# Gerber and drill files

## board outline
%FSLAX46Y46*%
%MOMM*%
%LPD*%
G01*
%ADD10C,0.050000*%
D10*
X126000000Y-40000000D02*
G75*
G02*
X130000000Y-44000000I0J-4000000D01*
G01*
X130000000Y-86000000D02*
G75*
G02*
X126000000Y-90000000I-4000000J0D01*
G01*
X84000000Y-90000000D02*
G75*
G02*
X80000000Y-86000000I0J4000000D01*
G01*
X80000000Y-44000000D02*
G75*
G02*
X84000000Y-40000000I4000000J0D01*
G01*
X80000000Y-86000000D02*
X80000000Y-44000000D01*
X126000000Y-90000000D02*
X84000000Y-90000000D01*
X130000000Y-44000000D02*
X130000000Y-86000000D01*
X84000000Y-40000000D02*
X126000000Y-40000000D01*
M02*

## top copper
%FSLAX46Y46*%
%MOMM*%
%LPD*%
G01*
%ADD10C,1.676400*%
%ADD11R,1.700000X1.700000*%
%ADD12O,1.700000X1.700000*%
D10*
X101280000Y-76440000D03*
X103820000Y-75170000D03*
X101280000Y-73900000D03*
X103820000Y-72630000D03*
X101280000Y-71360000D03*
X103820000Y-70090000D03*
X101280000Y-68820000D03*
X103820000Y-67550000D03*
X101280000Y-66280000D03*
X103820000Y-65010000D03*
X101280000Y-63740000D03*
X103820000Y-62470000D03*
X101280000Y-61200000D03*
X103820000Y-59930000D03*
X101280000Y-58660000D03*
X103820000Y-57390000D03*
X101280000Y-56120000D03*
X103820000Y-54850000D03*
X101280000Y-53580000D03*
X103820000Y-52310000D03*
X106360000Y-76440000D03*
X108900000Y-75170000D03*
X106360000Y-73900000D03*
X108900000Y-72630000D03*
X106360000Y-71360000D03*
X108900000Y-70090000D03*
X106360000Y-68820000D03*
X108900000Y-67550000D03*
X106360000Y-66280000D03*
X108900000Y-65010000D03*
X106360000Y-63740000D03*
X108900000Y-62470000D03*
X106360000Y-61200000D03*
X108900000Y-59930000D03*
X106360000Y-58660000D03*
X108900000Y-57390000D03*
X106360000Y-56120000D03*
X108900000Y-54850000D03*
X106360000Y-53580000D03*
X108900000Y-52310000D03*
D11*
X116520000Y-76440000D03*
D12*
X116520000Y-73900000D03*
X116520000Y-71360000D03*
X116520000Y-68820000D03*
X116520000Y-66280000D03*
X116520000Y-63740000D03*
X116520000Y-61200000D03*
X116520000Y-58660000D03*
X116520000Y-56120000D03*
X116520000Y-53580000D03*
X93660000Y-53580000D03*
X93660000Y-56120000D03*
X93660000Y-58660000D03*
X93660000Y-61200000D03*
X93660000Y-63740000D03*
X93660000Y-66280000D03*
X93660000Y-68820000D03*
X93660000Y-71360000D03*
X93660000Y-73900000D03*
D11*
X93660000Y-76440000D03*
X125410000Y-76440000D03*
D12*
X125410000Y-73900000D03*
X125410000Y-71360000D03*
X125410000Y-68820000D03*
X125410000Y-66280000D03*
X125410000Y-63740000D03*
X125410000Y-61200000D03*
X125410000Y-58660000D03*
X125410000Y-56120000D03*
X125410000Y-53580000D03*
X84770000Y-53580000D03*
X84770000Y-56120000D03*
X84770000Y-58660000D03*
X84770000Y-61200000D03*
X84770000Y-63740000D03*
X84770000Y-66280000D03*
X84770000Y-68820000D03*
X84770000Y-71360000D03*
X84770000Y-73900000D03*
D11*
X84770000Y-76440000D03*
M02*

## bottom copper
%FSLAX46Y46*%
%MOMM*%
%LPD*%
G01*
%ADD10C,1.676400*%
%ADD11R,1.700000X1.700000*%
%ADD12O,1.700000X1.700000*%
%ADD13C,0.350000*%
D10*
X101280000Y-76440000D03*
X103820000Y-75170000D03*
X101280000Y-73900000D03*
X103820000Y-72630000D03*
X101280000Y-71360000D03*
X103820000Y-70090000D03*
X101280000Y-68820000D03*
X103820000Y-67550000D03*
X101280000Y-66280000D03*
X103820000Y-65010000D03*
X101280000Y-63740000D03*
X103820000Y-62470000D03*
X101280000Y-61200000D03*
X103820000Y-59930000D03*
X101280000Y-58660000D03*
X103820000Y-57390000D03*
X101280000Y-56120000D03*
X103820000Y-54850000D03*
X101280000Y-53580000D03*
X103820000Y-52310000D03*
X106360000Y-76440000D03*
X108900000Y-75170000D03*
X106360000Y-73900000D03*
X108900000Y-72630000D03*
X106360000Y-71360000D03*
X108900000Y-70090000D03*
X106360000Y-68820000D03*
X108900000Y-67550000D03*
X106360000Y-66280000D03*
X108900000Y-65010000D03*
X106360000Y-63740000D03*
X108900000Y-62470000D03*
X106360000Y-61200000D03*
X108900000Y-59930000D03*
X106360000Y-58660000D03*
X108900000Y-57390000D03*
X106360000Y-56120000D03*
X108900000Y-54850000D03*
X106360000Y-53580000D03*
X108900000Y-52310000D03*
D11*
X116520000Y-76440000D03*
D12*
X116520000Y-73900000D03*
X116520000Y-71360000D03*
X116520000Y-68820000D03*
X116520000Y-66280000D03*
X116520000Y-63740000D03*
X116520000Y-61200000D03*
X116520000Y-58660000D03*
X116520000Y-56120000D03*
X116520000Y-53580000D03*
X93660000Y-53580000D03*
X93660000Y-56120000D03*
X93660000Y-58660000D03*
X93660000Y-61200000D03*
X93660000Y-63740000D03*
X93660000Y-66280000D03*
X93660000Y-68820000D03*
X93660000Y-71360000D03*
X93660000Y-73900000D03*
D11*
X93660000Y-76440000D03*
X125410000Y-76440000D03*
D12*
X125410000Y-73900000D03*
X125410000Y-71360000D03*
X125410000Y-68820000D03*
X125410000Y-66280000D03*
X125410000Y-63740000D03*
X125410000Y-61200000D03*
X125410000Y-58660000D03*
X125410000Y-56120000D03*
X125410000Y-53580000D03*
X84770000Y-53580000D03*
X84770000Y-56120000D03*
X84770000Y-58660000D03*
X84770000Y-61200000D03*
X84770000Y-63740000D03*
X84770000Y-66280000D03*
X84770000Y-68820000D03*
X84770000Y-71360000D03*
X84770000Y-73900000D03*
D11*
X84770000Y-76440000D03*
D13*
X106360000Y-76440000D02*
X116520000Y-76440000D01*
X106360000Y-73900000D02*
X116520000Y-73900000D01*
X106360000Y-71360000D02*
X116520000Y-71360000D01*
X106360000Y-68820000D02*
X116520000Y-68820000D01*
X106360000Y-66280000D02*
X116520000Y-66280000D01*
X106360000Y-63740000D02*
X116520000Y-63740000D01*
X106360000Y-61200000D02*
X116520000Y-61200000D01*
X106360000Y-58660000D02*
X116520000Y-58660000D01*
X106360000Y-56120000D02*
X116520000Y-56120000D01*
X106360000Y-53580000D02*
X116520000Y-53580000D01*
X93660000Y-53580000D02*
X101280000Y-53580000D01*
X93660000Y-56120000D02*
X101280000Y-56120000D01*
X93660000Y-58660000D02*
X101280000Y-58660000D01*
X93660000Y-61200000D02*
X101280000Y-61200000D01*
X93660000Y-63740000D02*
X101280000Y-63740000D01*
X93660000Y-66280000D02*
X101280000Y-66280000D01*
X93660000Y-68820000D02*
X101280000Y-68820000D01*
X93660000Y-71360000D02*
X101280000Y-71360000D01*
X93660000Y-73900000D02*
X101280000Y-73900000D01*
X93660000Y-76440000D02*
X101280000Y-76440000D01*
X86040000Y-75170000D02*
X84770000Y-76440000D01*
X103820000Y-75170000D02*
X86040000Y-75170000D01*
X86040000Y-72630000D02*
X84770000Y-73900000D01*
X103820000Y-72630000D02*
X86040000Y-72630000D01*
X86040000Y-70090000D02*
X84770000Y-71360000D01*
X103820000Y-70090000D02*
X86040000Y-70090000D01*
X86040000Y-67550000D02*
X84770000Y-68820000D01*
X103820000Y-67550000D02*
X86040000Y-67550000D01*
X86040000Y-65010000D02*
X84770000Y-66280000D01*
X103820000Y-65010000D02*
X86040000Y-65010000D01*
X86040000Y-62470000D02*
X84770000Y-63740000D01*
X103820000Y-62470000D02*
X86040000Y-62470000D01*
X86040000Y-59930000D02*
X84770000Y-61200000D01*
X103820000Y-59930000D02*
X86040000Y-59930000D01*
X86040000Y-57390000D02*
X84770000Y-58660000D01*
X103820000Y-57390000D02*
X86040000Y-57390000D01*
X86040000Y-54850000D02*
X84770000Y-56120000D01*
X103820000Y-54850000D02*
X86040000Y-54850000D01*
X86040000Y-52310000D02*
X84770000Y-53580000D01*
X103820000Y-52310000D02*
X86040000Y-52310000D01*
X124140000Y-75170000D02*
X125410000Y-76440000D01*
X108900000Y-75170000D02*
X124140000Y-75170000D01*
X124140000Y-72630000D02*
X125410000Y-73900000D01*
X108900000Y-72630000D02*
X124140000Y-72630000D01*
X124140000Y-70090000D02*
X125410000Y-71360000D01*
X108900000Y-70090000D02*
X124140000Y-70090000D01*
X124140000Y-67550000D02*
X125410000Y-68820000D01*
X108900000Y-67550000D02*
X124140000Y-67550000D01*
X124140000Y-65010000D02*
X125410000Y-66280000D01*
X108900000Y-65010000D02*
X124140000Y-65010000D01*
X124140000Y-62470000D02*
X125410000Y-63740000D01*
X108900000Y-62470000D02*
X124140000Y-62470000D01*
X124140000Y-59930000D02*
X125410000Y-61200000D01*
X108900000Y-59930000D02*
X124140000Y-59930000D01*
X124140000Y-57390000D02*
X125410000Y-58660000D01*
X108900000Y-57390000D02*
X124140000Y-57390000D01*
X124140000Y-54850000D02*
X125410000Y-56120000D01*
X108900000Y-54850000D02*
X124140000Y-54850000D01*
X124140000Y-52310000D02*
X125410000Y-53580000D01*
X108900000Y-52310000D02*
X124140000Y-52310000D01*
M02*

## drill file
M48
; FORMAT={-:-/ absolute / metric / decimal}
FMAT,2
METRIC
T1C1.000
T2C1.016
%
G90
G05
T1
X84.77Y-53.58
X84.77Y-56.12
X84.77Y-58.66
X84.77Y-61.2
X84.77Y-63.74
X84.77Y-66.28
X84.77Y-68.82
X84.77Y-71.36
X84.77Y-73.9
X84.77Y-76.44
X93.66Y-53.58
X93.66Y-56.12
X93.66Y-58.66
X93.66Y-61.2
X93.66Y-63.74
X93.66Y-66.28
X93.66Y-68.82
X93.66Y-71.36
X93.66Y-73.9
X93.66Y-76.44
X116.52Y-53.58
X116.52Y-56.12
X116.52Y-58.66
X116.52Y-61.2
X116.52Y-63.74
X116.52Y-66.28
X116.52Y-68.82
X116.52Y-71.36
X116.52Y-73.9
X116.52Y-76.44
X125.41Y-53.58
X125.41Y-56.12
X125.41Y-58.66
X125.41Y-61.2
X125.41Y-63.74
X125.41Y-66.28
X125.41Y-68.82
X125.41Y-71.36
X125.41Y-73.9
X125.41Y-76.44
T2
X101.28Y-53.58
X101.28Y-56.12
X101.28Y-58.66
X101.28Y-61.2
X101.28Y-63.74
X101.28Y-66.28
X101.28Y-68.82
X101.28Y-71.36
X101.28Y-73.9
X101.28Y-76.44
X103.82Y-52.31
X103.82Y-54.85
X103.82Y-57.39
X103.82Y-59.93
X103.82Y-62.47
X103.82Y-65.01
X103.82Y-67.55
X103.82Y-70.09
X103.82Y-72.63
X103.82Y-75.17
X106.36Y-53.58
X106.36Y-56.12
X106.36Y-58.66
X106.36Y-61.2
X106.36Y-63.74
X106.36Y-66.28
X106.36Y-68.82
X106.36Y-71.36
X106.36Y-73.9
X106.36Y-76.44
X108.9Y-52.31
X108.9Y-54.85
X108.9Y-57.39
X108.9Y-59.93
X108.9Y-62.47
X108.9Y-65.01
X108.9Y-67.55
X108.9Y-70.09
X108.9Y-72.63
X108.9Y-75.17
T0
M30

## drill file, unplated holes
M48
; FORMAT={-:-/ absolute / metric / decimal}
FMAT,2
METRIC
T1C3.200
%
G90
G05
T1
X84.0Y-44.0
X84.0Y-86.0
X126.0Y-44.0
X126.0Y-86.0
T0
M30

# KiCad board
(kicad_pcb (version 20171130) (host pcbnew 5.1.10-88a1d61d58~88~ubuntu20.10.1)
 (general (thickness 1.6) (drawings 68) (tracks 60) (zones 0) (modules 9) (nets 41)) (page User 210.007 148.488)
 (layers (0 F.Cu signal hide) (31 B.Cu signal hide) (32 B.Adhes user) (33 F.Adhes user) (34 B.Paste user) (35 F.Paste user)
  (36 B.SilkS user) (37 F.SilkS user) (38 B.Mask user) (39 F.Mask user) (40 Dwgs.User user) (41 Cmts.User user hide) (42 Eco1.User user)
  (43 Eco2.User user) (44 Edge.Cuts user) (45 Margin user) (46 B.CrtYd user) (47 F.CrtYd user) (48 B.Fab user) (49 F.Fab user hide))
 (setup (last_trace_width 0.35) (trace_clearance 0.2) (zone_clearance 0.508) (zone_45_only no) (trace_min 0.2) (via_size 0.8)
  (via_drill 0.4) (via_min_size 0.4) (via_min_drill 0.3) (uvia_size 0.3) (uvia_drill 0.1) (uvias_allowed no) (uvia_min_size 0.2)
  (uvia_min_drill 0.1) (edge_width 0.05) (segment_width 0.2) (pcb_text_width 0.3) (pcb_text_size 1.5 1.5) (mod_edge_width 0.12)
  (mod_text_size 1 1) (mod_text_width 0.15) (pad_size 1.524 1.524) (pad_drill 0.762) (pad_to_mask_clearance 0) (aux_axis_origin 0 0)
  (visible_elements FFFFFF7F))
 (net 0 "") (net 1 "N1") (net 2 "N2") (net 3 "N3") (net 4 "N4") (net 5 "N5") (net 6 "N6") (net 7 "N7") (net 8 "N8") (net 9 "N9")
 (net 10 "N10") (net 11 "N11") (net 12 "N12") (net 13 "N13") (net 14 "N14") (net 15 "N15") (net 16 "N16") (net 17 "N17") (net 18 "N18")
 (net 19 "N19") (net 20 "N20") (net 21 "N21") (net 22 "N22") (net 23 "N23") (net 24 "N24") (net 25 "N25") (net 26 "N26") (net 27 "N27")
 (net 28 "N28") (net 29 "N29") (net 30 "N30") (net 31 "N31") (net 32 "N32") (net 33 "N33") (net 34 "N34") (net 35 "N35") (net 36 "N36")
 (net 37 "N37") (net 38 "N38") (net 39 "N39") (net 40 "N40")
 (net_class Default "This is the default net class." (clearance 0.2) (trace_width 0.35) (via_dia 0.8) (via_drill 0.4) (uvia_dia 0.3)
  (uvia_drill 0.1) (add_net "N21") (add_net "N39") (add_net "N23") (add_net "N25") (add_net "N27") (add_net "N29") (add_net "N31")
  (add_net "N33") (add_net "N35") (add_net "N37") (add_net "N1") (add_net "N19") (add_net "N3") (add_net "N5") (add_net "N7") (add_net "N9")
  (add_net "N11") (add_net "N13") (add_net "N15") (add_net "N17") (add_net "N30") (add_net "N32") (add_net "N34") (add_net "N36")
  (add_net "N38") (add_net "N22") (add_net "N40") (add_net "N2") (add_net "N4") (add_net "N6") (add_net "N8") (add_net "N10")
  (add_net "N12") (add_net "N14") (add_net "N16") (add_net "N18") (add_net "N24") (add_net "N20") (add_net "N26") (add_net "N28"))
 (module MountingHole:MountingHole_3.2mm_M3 (layer F.Cu) (at 84 44)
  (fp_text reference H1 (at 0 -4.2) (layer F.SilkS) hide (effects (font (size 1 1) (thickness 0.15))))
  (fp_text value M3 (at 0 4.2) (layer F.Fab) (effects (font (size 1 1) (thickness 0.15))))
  (pad 1 np_thru_hole circle (at 0 0) (size 3.2 3.2) (drill 3.2) (layers *.Cu *.Mask)))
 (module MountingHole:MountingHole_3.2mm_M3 (layer F.Cu) (at 126 44)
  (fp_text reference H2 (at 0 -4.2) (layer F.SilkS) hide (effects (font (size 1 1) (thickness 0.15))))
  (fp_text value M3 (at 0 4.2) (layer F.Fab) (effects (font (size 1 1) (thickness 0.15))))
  (pad 1 np_thru_hole circle (at 0 0) (size 3.2 3.2) (drill 3.2) (layers *.Cu *.Mask)))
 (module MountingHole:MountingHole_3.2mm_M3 (layer F.Cu) (at 126 86)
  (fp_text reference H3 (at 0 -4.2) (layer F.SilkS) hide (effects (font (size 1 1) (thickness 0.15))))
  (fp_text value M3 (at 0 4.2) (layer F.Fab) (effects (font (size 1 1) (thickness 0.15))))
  (pad 1 np_thru_hole circle (at 0 0) (size 3.2 3.2) (drill 3.2) (layers *.Cu *.Mask)))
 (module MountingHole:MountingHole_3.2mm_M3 (layer F.Cu) (at 84 86)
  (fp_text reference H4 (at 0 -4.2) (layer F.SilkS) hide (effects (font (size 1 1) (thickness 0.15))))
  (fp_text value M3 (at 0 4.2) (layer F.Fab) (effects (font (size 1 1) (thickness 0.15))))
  (pad 1 np_thru_hole circle (at 0 0) (size 3.2 3.2) (drill 3.2) (layers *.Cu *.Mask)))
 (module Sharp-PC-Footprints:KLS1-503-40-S (layer F.Cu) (at 105.09 64.375 90)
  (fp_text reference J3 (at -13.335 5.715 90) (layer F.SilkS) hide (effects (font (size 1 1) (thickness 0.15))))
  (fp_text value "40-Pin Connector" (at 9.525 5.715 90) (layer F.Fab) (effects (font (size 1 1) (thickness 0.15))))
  (pad 21 thru_hole circle (at -12.065 -3.81 90) (size 1.6764 1.6764) (drill 1.016) (layers *.Cu *.Mask) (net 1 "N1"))
  (pad 22 thru_hole circle (at -10.795 -1.27 90) (size 1.6764 1.6764) (drill 1.016) (layers *.Cu *.Mask) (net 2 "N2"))
  (pad 23 thru_hole circle (at -9.525 -3.81 90) (size 1.6764 1.6764) (drill 1.016) (layers *.Cu *.Mask) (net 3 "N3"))
  (pad 24 thru_hole circle (at -8.255 -1.27 90) (size 1.6764 1.6764) (drill 1.016) (layers *.Cu *.Mask) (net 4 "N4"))
  (pad 25 thru_hole circle (at -6.985 -3.81 90) (size 1.6764 1.6764) (drill 1.016) (layers *.Cu *.Mask) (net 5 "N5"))
  (pad 26 thru_hole circle (at -5.715 -1.27 90) (size 1.6764 1.6764) (drill 1.016) (layers *.Cu *.Mask) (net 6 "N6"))
  (pad 27 thru_hole circle (at -4.445 -3.81 90) (size 1.6764 1.6764) (drill 1.016) (layers *.Cu *.Mask) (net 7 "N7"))
  (pad 28 thru_hole circle (at -3.175 -1.27 90) (size 1.6764 1.6764) (drill 1.016) (layers *.Cu *.Mask) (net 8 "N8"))
  (pad 29 thru_hole circle (at -1.905 -3.81 90) (size 1.6764 1.6764) (drill 1.016) (layers *.Cu *.Mask) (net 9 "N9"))
  (pad 30 thru_hole circle (at -0.635 -1.27 90) (size 1.6764 1.6764) (drill 1.016) (layers *.Cu *.Mask) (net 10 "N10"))
  (pad 31 thru_hole circle (at 0.635 -3.81 90) (size 1.6764 1.6764) (drill 1.016) (layers *.Cu *.Mask) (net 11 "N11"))
  (pad 32 thru_hole circle (at 1.905 -1.27 90) (size 1.6764 1.6764) (drill 1.016) (layers *.Cu *.Mask) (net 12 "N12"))
  (pad 33 thru_hole circle (at 3.175 -3.81 90) (size 1.6764 1.6764) (drill 1.016) (layers *.Cu *.Mask) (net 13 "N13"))
  (pad 34 thru_hole circle (at 4.445 -1.27 90) (size 1.6764 1.6764) (drill 1.016) (layers *.Cu *.Mask) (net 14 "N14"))
  (pad 35 thru_hole circle (at 5.715 -3.81 90) (size 1.6764 1.6764) (drill 1.016) (layers *.Cu *.Mask) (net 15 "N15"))
  (pad 36 thru_hole circle (at 6.985 -1.27 90) (size 1.6764 1.6764) (drill 1.016) (layers *.Cu *.Mask) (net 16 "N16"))
  (pad 37 thru_hole circle (at 8.255 -3.81 90) (size 1.6764 1.6764) (drill 1.016) (layers *.Cu *.Mask) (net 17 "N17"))
  (pad 38 thru_hole circle (at 9.525 -1.27 90) (size 1.6764 1.6764) (drill 1.016) (layers *.Cu *.Mask) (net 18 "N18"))
  (pad 39 thru_hole circle (at 10.795 -3.81 90) (size 1.6764 1.6764) (drill 1.016) (layers *.Cu *.Mask) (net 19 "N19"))
  (pad 40 thru_hole circle (at 12.065 -1.27 90) (size 1.6764 1.6764) (drill 1.016) (layers *.Cu *.Mask) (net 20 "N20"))
  (pad 1 thru_hole circle (at -12.065 1.27 90) (size 1.6764 1.6764) (drill 1.016) (layers *.Cu *.Mask) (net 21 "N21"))
  (pad 2 thru_hole circle (at -10.795 3.81 90) (size 1.6764 1.6764) (drill 1.016) (layers *.Cu *.Mask) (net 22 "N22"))
  (pad 3 thru_hole circle (at -9.525 1.27 90) (size 1.6764 1.6764) (drill 1.016) (layers *.Cu *.Mask) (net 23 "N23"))
  (pad 4 thru_hole circle (at -8.255 3.81 90) (size 1.6764 1.6764) (drill 1.016) (layers *.Cu *.Mask) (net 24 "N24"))
  (pad 5 thru_hole circle (at -6.985 1.27 180) (size 1.6764 1.6764) (drill 1.016) (layers *.Cu *.Mask) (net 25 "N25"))
  (pad 6 thru_hole circle (at -5.715 3.81 90) (size 1.6764 1.6764) (drill 1.016) (layers *.Cu *.Mask) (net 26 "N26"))
  (pad 7 thru_hole circle (at -4.445 1.27 90) (size 1.6764 1.6764) (drill 1.016) (layers *.Cu *.Mask) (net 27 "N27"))
  (pad 8 thru_hole circle (at -3.175 3.81 90) (size 1.6764 1.6764) (drill 1.016) (layers *.Cu *.Mask) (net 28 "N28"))
  (pad 9 thru_hole circle (at -1.905 1.27 90) (size 1.6764 1.6764) (drill 1.016) (layers *.Cu *.Mask) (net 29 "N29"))
  (pad 10 thru_hole circle (at -0.635 3.81 90) (size 1.6764 1.6764) (drill 1.016) (layers *.Cu *.Mask) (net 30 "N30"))
  (pad 11 thru_hole circle (at 0.635 1.27 90) (size 1.6764 1.6764) (drill 1.016) (layers *.Cu *.Mask) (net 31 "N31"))
  (pad 12 thru_hole circle (at 1.905 3.81 90) (size 1.6764 1.6764) (drill 1.016) (layers *.Cu *.Mask) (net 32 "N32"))
  (pad 13 thru_hole circle (at 3.175 1.27 90) (size 1.6764 1.6764) (drill 1.016) (layers *.Cu *.Mask) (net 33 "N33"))
  (pad 14 thru_hole circle (at 4.445 3.81 90) (size 1.6764 1.6764) (drill 1.016) (layers *.Cu *.Mask) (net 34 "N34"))
  (pad 15 thru_hole circle (at 5.715 1.27 90) (size 1.6764 1.6764) (drill 1.016) (layers *.Cu *.Mask) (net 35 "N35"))
  (pad 16 thru_hole circle (at 6.985 3.81 90) (size 1.6764 1.6764) (drill 1.016) (layers *.Cu *.Mask) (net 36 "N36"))
  (pad 17 thru_hole circle (at 8.255 1.27 90) (size 1.6764 1.6764) (drill 1.016) (layers *.Cu *.Mask) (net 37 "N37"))
  (pad 18 thru_hole circle (at 9.525 3.81 90) (size 1.6764 1.6764) (drill 1.016) (layers *.Cu *.Mask) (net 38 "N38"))
  (pad 19 thru_hole circle (at 10.795 1.27 90) (size 1.6764 1.6764) (drill 1.016) (layers *.Cu *.Mask) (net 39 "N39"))
  (pad 20 thru_hole circle (at 12.065 3.81 90) (size 1.6764 1.6764) (drill 1.016) (layers *.Cu *.Mask) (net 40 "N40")))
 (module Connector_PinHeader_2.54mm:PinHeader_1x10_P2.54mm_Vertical (layer F.Cu) (at 116.52 76.44 180)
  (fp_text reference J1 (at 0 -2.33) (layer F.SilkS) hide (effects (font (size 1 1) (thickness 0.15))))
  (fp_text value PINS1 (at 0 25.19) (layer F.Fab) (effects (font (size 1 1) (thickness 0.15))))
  (pad 1 thru_hole rect (at 0 0 180) (size 1.7 1.7) (drill 1) (layers *.Cu *.Mask) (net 21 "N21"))
  (pad 2 thru_hole oval (at 0 2.54 180) (size 1.7 1.7) (drill 1) (layers *.Cu *.Mask) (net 23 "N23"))
  (pad 3 thru_hole oval (at 0 5.08 180) (size 1.7 1.7) (drill 1) (layers *.Cu *.Mask) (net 25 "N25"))
  (pad 4 thru_hole oval (at 0 7.62 180) (size 1.7 1.7) (drill 1) (layers *.Cu *.Mask) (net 27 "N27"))
  (pad 5 thru_hole oval (at 0 10.16 180) (size 1.7 1.7) (drill 1) (layers *.Cu *.Mask) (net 29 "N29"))
  (pad 6 thru_hole oval (at 0 12.7 180) (size 1.7 1.7) (drill 1) (layers *.Cu *.Mask) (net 31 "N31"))
  (pad 7 thru_hole oval (at 0 15.24 180) (size 1.7 1.7) (drill 1) (layers *.Cu *.Mask) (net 33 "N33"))
  (pad 8 thru_hole oval (at 0 17.78 180) (size 1.7 1.7) (drill 1) (layers *.Cu *.Mask) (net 35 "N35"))
  (pad 9 thru_hole oval (at 0 20.32 180) (size 1.7 1.7) (drill 1) (layers *.Cu *.Mask) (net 37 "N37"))
  (pad 10 thru_hole oval (at 0 22.86 180) (size 1.7 1.7) (drill 1) (layers *.Cu *.Mask) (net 39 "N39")))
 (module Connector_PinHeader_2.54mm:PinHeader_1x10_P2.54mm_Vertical (layer F.Cu) (at 93.66 76.44 180)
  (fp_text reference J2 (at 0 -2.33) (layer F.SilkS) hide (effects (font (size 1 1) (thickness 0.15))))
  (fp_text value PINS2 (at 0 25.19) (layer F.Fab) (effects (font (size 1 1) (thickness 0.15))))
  (pad 10 thru_hole oval (at 0 22.86 180) (size 1.7 1.7) (drill 1) (layers *.Cu *.Mask) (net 19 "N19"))
  (pad 9 thru_hole oval (at 0 20.32 180) (size 1.7 1.7) (drill 1) (layers *.Cu *.Mask) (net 17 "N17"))
  (pad 8 thru_hole oval (at 0 17.78 180) (size 1.7 1.7) (drill 1) (layers *.Cu *.Mask) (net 15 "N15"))
  (pad 7 thru_hole oval (at 0 15.24 180) (size 1.7 1.7) (drill 1) (layers *.Cu *.Mask) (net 13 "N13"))
  (pad 6 thru_hole oval (at 0 12.7 180) (size 1.7 1.7) (drill 1) (layers *.Cu *.Mask) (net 11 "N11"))
  (pad 5 thru_hole oval (at 0 10.16 180) (size 1.7 1.7) (drill 1) (layers *.Cu *.Mask) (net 9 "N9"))
  (pad 4 thru_hole oval (at 0 7.62 180) (size 1.7 1.7) (drill 1) (layers *.Cu *.Mask) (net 7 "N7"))
  (pad 3 thru_hole oval (at 0 5.08 180) (size 1.7 1.7) (drill 1) (layers *.Cu *.Mask) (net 5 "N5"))
  (pad 2 thru_hole oval (at 0 2.54 180) (size 1.7 1.7) (drill 1) (layers *.Cu *.Mask) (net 3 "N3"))
  (pad 1 thru_hole rect (at 0 0 180) (size 1.7 1.7) (drill 1) (layers *.Cu *.Mask) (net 1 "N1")))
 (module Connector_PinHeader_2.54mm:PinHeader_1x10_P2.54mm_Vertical (layer F.Cu) (at 125.41 76.44 180)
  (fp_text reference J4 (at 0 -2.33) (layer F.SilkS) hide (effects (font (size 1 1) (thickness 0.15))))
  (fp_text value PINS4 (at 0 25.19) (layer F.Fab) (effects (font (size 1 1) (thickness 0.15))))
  (pad 1 thru_hole rect (at 0 0 180) (size 1.7 1.7) (drill 1) (layers *.Cu *.Mask) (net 22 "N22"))
  (pad 2 thru_hole oval (at 0 2.54 180) (size 1.7 1.7) (drill 1) (layers *.Cu *.Mask) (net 24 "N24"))
  (pad 3 thru_hole oval (at 0 5.08 180) (size 1.7 1.7) (drill 1) (layers *.Cu *.Mask) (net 26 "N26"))
  (pad 4 thru_hole oval (at 0 7.62 180) (size 1.7 1.7) (drill 1) (layers *.Cu *.Mask) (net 28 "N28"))
  (pad 5 thru_hole oval (at 0 10.16 180) (size 1.7 1.7) (drill 1) (layers *.Cu *.Mask) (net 30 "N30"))
  (pad 6 thru_hole oval (at 0 12.7 180) (size 1.7 1.7) (drill 1) (layers *.Cu *.Mask) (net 32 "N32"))
  (pad 7 thru_hole oval (at 0 15.24 180) (size 1.7 1.7) (drill 1) (layers *.Cu *.Mask) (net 34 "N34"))
  (pad 8 thru_hole oval (at 0 17.78 180) (size 1.7 1.7) (drill 1) (layers *.Cu *.Mask) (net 36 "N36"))
  (pad 9 thru_hole oval (at 0 20.32 180) (size 1.7 1.7) (drill 1) (layers *.Cu *.Mask) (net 38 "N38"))
  (pad 10 thru_hole oval (at 0 22.86 180) (size 1.7 1.7) (drill 1) (layers *.Cu *.Mask) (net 40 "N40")))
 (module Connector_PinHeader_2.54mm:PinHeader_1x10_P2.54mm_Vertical (layer F.Cu) (at 84.77 76.44 180)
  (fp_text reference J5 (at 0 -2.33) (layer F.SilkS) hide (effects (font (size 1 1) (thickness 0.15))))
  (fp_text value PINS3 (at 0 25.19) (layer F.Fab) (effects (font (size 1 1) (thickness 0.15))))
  (pad 10 thru_hole oval (at 0 22.86 180) (size 1.7 1.7) (drill 1) (layers *.Cu *.Mask) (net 20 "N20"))
  (pad 9 thru_hole oval (at 0 20.32 180) (size 1.7 1.7) (drill 1) (layers *.Cu *.Mask) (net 18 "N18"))
  (pad 8 thru_hole oval (at 0 17.78 180) (size 1.7 1.7) (drill 1) (layers *.Cu *.Mask) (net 16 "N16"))
  (pad 7 thru_hole oval (at 0 15.24 180) (size 1.7 1.7) (drill 1) (layers *.Cu *.Mask) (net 14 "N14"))
  (pad 6 thru_hole oval (at 0 12.7 180) (size 1.7 1.7) (drill 1) (layers *.Cu *.Mask) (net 12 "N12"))
  (pad 5 thru_hole oval (at 0 10.16 180) (size 1.7 1.7) (drill 1) (layers *.Cu *.Mask) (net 10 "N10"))
  (pad 4 thru_hole oval (at 0 7.62 180) (size 1.7 1.7) (drill 1) (layers *.Cu *.Mask) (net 8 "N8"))
  (pad 3 thru_hole oval (at 0 5.08 180) (size 1.7 1.7) (drill 1) (layers *.Cu *.Mask) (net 6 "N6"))
  (pad 2 thru_hole oval (at 0 2.54 180) (size 1.7 1.7) (drill 1) (layers *.Cu *.Mask) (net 4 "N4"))
  (pad 1 thru_hole rect (at 0 0 180) (size 1.7 1.7) (drill 1) (layers *.Cu *.Mask) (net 2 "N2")))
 (gr_arc (start 126 44) (end 130 44) (angle -90) (layer Edge.Cuts) (width 0.05))
 (gr_arc (start 126 86) (end 126 90) (angle -90) (layer Edge.Cuts) (width 0.05))
 (gr_arc (start 84 86) (end 80 86) (angle -90) (layer Edge.Cuts) (width 0.05))
 (gr_arc (start 84 44) (end 84 40) (angle -90) (layer Edge.Cuts) (width 0.05))
 (gr_line (start 80 86) (end 80 44) (layer Edge.Cuts) (width 0.05))
 (gr_line (start 126 90) (end 84 90) (layer Edge.Cuts) (width 0.05))
 (gr_line (start 130 44) (end 130 86) (layer Edge.Cuts) (width 0.05))
 (gr_line (start 84 40) (end 126 40) (layer Edge.Cuts) (width 0.05))
 (segment (start 106.36 76.44) (end 116.52 76.44) (width 0.35) (layer B.Cu) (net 21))
 (segment (start 106.36 73.9) (end 116.52 73.9) (width 0.35) (layer B.Cu) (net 23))
 (segment (start 106.36 71.36) (end 116.52 71.36) (width 0.35) (layer B.Cu) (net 25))
 (segment (start 106.36 68.82) (end 116.52 68.82) (width 0.35) (layer B.Cu) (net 27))
 (segment (start 106.36 66.28) (end 116.52 66.28) (width 0.35) (layer B.Cu) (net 29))
 (segment (start 106.36 63.74) (end 116.52 63.74) (width 0.35) (layer B.Cu) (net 31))
 (segment (start 106.36 61.2) (end 116.52 61.2) (width 0.35) (layer B.Cu) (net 33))
 (segment (start 106.36 58.66) (end 116.52 58.66) (width 0.35) (layer B.Cu) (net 35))
 (segment (start 106.36 56.12) (end 116.52 56.12) (width 0.35) (layer B.Cu) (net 37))
 (segment (start 106.36 53.58) (end 116.52 53.58) (width 0.35) (layer B.Cu) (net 39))
 (segment (start 93.66 53.58) (end 101.28 53.58) (width 0.35) (layer B.Cu) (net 19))
 (segment (start 93.66 56.12) (end 101.28 56.12) (width 0.35) (layer B.Cu) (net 17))
 (segment (start 93.66 58.66) (end 101.28 58.66) (width 0.35) (layer B.Cu) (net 15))
 (segment (start 93.66 61.2) (end 101.28 61.2) (width 0.35) (layer B.Cu) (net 13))
 (segment (start 93.66 63.74) (end 101.28 63.74) (width 0.35) (layer B.Cu) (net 11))
 (segment (start 93.66 66.28) (end 101.28 66.28) (width 0.35) (layer B.Cu) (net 9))
 (segment (start 93.66 68.82) (end 101.28 68.82) (width 0.35) (layer B.Cu) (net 7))
 (segment (start 93.66 71.36) (end 101.28 71.36) (width 0.35) (layer B.Cu) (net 5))
 (segment (start 93.66 73.9) (end 101.28 73.9) (width 0.35) (layer B.Cu) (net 3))
 (segment (start 93.66 76.44) (end 101.28 76.44) (width 0.35) (layer B.Cu) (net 1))
 (segment (start 86.04 75.17) (end 84.77 76.44) (width 0.35) (layer B.Cu) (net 2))
 (segment (start 103.82 75.17) (end 86.04 75.17) (width 0.35) (layer B.Cu) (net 2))
 (segment (start 86.04 72.63) (end 84.77 73.9) (width 0.35) (layer B.Cu) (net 4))
 (segment (start 103.82 72.63) (end 86.04 72.63) (width 0.35) (layer B.Cu) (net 4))
 (segment (start 86.04 70.09) (end 84.77 71.36) (width 0.35) (layer B.Cu) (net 6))
 (segment (start 103.82 70.09) (end 86.04 70.09) (width 0.35) (layer B.Cu) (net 6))
 (segment (start 86.04 67.55) (end 84.77 68.82) (width 0.35) (layer B.Cu) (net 8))
 (segment (start 103.82 67.55) (end 86.04 67.55) (width 0.35) (layer B.Cu) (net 8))
 (segment (start 86.04 65.01) (end 84.77 66.28) (width 0.35) (layer B.Cu) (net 10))
 (segment (start 103.82 65.01) (end 86.04 65.01) (width 0.35) (layer B.Cu) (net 10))
 (segment (start 86.04 62.47) (end 84.77 63.74) (width 0.35) (layer B.Cu) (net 12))
 (segment (start 103.82 62.47) (end 86.04 62.47) (width 0.35) (layer B.Cu) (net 12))
 (segment (start 86.04 59.93) (end 84.77 61.2) (width 0.35) (layer B.Cu) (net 14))
 (segment (start 103.82 59.93) (end 86.04 59.93) (width 0.35) (layer B.Cu) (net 14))
 (segment (start 86.04 57.39) (end 84.77 58.66) (width 0.35) (layer B.Cu) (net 16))
 (segment (start 103.82 57.39) (end 86.04 57.39) (width 0.35) (layer B.Cu) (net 16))
 (segment (start 86.04 54.85) (end 84.77 56.12) (width 0.35) (layer B.Cu) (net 18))
 (segment (start 103.82 54.85) (end 86.04 54.85) (width 0.35) (layer B.Cu) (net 18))
 (segment (start 86.04 52.31) (end 84.77 53.58) (width 0.35) (layer B.Cu) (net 20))
 (segment (start 103.82 52.31) (end 86.04 52.31) (width 0.35) (layer B.Cu) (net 20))
 (segment (start 124.14 75.17) (end 125.41 76.44) (width 0.35) (layer B.Cu) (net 22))
 (segment (start 108.9 75.17) (end 124.14 75.17) (width 0.35) (layer B.Cu) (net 22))
 (segment (start 124.14 72.63) (end 125.41 73.9) (width 0.35) (layer B.Cu) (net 24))
 (segment (start 108.9 72.63) (end 124.14 72.63) (width 0.35) (layer B.Cu) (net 24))
 (segment (start 124.14 70.09) (end 125.41 71.36) (width 0.35) (layer B.Cu) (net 26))
 (segment (start 108.9 70.09) (end 124.14 70.09) (width 0.35) (layer B.Cu) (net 26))
 (segment (start 124.14 67.55) (end 125.41 68.82) (width 0.35) (layer B.Cu) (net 28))
 (segment (start 108.9 67.55) (end 124.14 67.55) (width 0.35) (layer B.Cu) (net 28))
 (segment (start 124.14 65.01) (end 125.41 66.28) (width 0.35) (layer B.Cu) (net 30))
 (segment (start 108.9 65.01) (end 124.14 65.01) (width 0.35) (layer B.Cu) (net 30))
 (segment (start 124.14 62.47) (end 125.41 63.74) (width 0.35) (layer B.Cu) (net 32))
 (segment (start 108.9 62.47) (end 124.14 62.47) (width 0.35) (layer B.Cu) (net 32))
 (segment (start 124.14 59.93) (end 125.41 61.2) (width 0.35) (layer B.Cu) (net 34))
 (segment (start 108.9 59.93) (end 124.14 59.93) (width 0.35) (layer B.Cu) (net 34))
 (segment (start 124.14 57.39) (end 125.41 58.66) (width 0.35) (layer B.Cu) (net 36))
 (segment (start 108.9 57.39) (end 124.14 57.39) (width 0.35) (layer B.Cu) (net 36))
 (segment (start 124.14 54.85) (end 125.41 56.12) (width 0.35) (layer B.Cu) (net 38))
 (segment (start 108.9 54.85) (end 124.14 54.85) (width 0.35) (layer B.Cu) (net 38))
 (segment (start 124.14 52.31) (end 125.41 53.58) (width 0.35) (layer B.Cu) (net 40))
 (segment (start 108.9 52.31) (end 124.14 52.31) (width 0.35) (layer B.Cu) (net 40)))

